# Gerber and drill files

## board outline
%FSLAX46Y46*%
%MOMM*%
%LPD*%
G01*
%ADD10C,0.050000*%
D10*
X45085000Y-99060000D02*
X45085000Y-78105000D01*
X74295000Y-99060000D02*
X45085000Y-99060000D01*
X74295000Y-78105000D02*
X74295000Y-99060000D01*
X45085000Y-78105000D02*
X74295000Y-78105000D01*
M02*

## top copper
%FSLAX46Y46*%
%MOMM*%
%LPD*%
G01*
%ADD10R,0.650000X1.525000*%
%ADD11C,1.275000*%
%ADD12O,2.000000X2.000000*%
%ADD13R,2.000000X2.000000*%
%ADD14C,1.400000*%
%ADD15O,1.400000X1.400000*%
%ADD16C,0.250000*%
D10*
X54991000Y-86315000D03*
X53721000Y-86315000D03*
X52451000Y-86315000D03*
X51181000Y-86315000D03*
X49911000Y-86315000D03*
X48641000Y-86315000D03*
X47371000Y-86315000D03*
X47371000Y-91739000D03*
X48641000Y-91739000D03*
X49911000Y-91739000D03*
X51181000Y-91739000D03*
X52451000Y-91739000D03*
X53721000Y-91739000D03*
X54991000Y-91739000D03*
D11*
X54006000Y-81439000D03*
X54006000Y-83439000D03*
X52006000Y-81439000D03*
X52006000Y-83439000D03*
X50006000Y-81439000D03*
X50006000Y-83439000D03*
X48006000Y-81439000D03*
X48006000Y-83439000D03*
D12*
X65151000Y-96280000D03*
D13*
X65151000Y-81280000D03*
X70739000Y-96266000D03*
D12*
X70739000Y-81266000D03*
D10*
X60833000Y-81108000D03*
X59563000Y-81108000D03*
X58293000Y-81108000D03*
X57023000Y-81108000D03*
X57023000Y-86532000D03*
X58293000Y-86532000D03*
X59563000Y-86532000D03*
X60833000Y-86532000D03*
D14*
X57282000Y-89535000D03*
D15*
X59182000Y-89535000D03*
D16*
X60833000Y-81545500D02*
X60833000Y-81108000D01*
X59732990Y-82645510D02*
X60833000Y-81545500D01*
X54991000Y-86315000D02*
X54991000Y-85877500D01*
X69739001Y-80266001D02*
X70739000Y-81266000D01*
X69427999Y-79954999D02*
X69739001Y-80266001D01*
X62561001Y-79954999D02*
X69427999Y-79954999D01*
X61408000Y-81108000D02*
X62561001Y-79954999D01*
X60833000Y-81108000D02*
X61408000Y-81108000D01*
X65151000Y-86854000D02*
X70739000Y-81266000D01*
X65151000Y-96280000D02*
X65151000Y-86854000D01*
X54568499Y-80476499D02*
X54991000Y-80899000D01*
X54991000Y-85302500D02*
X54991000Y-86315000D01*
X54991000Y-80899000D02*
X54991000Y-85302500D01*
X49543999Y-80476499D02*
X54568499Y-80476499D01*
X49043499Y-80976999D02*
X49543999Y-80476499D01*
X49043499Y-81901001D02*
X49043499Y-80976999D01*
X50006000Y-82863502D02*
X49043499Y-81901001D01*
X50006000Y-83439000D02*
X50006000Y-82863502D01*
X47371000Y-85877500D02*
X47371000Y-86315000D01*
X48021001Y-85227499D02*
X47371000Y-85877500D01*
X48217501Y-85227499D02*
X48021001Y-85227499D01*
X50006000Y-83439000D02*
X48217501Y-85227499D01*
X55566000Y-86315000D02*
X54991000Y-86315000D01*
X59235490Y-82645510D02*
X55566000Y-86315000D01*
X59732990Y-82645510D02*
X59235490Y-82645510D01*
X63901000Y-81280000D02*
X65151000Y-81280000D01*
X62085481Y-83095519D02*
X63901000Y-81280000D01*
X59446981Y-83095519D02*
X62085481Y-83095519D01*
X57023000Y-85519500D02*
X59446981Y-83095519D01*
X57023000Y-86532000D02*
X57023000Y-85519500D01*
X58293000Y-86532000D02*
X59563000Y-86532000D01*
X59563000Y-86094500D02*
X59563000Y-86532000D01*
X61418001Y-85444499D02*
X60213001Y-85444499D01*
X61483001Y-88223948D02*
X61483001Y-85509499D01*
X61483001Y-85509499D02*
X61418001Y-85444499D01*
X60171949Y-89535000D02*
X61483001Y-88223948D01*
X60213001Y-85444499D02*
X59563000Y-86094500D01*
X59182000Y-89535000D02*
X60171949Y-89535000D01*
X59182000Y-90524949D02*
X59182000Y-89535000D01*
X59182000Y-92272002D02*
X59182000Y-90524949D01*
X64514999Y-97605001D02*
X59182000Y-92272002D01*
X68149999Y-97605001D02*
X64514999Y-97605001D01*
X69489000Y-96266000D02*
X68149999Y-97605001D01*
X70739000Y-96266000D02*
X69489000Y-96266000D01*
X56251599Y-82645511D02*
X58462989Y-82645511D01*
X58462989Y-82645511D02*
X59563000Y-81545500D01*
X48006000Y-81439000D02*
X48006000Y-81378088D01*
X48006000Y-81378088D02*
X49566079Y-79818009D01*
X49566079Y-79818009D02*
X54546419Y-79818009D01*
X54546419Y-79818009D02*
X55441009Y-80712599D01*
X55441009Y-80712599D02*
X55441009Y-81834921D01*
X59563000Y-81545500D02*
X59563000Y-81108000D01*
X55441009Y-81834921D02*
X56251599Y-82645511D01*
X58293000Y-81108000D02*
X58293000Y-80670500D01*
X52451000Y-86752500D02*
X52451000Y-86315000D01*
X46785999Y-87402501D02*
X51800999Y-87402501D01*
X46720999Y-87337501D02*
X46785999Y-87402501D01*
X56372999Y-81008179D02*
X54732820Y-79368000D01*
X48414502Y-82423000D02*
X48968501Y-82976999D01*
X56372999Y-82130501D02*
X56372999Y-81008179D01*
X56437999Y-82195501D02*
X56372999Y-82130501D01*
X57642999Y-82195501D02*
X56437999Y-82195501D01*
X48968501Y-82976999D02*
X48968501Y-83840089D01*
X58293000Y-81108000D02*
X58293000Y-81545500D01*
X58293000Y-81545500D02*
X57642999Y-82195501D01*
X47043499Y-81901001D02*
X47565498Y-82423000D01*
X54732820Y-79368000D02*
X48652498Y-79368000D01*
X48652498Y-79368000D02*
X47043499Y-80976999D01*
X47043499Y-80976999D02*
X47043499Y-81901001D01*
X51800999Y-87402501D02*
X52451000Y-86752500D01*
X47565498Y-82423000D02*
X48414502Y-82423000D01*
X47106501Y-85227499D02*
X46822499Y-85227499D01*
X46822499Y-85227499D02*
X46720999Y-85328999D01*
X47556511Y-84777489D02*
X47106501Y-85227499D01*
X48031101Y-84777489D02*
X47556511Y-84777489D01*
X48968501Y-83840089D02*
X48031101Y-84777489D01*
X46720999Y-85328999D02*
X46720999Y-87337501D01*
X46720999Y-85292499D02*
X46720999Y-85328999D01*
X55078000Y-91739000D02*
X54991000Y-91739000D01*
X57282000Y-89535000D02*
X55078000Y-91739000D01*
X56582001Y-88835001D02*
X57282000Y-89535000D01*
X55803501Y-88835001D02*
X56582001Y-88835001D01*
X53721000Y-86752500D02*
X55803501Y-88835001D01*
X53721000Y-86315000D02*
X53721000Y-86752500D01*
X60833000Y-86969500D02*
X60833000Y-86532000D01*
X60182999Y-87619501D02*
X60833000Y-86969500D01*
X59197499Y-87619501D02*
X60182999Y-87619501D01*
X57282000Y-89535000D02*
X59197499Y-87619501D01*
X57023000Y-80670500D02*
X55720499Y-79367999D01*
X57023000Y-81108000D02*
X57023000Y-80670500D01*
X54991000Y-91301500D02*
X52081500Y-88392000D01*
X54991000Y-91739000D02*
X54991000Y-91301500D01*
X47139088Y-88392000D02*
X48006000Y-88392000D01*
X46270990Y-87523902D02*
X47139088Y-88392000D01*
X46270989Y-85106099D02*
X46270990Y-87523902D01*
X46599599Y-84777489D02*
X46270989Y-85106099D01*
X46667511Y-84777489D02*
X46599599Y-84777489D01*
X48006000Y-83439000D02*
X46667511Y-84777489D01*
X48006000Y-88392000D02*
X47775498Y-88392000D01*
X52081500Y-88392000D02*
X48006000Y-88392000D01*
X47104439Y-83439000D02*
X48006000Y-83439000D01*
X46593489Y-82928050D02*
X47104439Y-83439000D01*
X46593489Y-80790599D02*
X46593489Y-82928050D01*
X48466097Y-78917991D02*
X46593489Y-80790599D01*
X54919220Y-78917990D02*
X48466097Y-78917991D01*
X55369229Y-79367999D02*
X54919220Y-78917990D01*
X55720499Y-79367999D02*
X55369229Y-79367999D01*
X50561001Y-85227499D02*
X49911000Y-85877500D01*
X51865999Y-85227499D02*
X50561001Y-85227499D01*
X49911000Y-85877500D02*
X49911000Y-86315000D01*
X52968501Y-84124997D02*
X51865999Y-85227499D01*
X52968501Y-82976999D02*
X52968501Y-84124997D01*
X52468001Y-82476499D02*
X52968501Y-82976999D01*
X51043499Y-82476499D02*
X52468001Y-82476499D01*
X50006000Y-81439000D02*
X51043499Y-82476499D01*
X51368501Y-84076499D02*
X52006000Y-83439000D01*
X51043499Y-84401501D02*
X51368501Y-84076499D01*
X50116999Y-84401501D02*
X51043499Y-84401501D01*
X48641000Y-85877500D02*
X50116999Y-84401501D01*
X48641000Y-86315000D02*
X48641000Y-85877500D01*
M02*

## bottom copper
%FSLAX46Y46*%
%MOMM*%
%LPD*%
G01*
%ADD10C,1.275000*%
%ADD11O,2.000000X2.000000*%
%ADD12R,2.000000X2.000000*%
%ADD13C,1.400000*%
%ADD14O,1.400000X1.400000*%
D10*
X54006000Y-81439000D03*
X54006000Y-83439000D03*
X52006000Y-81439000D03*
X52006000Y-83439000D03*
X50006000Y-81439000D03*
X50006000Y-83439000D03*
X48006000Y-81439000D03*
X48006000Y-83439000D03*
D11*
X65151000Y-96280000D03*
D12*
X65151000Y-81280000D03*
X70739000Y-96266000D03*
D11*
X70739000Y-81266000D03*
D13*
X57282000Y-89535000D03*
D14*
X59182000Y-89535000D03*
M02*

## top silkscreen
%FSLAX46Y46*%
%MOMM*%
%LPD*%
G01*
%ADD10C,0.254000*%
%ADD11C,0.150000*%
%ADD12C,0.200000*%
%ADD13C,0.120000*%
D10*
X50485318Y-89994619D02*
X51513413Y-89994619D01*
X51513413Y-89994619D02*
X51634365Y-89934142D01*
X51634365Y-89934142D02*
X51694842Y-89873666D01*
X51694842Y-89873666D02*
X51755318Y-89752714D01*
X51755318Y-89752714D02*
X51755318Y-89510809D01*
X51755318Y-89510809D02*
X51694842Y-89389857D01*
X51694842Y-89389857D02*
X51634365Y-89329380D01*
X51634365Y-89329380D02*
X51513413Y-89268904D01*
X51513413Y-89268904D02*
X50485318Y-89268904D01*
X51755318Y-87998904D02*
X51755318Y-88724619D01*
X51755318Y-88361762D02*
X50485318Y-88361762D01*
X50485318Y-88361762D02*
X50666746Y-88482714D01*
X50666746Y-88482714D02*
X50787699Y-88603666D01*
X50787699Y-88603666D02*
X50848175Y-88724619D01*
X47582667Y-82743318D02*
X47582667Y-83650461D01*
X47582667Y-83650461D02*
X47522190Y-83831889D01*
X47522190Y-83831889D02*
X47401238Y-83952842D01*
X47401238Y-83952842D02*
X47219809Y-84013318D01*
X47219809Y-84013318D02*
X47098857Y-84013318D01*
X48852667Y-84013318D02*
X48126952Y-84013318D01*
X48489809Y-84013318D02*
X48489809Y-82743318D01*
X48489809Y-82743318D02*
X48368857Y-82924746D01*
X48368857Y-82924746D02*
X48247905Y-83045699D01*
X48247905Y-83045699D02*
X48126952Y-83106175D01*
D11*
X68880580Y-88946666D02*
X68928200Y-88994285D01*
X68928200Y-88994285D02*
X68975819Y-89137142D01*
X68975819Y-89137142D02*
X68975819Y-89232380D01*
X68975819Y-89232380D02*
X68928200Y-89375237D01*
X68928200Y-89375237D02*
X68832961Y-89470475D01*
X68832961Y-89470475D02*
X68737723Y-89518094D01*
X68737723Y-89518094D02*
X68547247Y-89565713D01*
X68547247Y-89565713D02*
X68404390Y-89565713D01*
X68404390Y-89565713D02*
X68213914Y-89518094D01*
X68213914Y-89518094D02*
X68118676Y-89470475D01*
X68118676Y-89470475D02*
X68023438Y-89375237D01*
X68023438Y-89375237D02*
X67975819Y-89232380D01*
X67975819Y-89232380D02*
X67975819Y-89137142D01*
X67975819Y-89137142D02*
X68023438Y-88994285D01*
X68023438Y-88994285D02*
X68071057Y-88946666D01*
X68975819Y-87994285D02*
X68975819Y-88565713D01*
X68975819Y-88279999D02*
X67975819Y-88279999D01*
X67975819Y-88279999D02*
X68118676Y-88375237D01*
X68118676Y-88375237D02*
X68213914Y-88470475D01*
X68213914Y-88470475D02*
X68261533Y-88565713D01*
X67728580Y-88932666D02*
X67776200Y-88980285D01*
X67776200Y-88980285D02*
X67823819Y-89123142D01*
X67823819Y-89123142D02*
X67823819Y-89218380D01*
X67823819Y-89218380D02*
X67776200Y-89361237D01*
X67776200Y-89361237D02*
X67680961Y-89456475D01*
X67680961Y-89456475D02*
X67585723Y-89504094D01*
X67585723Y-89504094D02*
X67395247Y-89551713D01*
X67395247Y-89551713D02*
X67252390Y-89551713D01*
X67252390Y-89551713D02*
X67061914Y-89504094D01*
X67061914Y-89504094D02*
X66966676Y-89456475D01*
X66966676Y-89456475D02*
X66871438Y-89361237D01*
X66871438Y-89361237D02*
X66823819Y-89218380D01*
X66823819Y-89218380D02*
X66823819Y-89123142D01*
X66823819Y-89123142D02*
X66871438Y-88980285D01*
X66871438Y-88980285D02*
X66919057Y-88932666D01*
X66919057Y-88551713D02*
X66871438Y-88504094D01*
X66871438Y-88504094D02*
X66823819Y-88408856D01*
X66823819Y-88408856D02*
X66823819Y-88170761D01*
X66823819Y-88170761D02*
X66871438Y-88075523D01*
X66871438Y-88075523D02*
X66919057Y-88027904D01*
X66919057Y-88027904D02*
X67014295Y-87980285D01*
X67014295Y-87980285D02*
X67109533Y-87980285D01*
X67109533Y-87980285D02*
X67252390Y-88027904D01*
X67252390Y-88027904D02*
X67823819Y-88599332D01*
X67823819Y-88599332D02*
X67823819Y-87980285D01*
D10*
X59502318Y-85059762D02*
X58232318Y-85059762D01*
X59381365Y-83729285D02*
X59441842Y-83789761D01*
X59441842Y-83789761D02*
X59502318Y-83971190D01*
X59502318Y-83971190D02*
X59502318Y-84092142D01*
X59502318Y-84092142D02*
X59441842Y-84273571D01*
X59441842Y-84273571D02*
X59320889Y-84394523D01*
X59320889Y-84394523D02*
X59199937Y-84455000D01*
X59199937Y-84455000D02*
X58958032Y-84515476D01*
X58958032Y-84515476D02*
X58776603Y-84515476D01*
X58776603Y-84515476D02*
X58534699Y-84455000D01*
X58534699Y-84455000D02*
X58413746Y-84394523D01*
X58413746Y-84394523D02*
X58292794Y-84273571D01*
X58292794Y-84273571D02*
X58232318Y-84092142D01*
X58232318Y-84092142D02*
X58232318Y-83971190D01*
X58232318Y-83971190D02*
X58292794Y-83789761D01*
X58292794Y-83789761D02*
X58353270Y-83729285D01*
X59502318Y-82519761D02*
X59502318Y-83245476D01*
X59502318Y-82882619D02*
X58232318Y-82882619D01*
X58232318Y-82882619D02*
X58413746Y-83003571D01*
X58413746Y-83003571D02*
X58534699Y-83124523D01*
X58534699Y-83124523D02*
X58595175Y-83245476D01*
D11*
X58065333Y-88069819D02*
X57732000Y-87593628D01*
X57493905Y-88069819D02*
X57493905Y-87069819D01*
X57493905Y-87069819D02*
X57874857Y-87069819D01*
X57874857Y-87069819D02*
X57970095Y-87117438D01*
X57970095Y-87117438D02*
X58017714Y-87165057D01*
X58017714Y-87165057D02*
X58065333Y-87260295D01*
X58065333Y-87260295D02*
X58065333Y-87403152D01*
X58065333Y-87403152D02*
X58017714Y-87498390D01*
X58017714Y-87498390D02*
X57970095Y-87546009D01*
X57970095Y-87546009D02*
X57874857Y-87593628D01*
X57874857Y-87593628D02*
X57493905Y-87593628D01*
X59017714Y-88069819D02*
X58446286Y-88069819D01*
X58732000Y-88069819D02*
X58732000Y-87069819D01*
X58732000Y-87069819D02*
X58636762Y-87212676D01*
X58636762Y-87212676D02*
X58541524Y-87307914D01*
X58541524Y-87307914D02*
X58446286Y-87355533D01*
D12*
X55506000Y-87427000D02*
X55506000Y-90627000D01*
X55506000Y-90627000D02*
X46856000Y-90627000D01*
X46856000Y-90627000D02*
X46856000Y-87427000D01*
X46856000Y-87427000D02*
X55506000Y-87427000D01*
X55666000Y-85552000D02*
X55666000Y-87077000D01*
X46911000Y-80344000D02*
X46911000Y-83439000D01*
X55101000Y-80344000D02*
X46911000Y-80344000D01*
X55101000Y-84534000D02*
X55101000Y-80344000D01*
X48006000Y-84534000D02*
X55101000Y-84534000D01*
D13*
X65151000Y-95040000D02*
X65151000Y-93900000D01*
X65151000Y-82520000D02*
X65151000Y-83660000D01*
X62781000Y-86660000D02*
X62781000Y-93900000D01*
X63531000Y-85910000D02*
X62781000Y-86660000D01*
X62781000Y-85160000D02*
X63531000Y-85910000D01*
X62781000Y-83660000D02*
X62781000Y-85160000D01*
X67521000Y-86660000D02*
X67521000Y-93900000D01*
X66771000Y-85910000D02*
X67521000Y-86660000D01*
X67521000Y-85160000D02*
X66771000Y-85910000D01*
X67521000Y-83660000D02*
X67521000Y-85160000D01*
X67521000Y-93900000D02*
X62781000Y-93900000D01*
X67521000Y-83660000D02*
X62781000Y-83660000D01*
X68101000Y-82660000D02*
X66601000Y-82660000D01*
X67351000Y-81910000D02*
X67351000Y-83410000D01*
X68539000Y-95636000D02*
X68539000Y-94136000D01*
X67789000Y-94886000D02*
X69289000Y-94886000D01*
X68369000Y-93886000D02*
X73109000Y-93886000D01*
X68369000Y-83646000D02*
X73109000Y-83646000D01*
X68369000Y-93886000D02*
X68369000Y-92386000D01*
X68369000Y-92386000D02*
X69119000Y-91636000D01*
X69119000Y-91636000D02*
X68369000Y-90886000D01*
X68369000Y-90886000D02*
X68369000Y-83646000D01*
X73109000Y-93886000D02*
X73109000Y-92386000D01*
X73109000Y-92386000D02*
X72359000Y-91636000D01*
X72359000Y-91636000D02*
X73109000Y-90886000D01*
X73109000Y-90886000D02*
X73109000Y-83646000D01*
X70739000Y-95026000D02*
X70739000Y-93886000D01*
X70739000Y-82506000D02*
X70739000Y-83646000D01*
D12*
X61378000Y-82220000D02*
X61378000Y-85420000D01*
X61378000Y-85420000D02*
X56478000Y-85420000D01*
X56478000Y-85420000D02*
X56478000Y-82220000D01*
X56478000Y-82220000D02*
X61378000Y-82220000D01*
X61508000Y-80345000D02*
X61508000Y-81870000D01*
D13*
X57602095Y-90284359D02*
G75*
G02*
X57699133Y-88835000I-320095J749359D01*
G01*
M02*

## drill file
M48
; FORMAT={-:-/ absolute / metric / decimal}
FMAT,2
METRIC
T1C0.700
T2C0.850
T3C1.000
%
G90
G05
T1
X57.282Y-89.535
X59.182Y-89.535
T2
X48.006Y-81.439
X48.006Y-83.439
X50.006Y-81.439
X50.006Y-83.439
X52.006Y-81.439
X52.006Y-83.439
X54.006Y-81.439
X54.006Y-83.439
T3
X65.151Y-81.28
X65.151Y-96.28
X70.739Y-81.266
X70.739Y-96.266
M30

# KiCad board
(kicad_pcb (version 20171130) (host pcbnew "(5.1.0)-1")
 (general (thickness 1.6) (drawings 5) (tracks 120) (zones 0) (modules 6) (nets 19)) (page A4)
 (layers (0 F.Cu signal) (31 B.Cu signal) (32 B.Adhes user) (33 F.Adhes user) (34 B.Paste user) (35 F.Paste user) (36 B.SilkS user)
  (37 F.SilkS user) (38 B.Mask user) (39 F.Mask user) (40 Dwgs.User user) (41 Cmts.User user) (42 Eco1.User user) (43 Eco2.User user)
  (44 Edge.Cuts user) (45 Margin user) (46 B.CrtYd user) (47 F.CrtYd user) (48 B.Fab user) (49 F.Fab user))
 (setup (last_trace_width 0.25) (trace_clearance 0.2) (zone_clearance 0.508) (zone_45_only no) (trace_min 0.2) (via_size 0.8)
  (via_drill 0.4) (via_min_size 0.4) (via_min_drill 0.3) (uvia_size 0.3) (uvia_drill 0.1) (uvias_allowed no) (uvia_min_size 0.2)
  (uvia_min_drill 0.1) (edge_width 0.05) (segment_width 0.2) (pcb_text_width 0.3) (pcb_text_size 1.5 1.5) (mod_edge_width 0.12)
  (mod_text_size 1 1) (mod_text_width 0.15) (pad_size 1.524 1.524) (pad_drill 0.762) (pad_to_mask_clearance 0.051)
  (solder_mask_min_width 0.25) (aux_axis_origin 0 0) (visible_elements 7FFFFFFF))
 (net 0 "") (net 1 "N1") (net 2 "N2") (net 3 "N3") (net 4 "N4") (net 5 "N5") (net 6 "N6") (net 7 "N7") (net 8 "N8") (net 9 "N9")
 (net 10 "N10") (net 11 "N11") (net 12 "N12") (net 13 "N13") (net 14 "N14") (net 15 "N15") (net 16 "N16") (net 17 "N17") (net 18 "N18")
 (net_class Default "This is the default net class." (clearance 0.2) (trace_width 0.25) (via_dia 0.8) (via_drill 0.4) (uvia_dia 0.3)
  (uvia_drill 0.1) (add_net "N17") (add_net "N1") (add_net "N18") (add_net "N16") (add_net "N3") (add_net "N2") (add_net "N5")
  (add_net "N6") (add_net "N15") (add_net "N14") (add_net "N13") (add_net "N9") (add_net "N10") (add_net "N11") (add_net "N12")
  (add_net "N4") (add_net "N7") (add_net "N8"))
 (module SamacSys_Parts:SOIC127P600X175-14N (layer F.Cu) (at 51.181 89.027 270)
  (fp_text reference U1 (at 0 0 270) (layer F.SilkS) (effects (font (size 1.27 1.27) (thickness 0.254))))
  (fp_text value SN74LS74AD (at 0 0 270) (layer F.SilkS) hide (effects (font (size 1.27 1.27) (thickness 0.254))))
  (fp_line (start -1.6 -4.325) (end 1.6 -4.325) (layer F.SilkS) (width 0.2))
  (fp_line (start 1.6 -4.325) (end 1.6 4.325) (layer F.SilkS) (width 0.2))
  (fp_line (start 1.6 4.325) (end -1.6 4.325) (layer F.SilkS) (width 0.2))
  (fp_line (start -1.6 4.325) (end -1.6 -4.325) (layer F.SilkS) (width 0.2))
  (fp_line (start -3.475 -4.485) (end -1.95 -4.485) (layer F.SilkS) (width 0.2))
  (pad 1 smd rect (at -2.712 -3.81) (size 0.65 1.525) (layers F.Cu F.Paste F.Mask) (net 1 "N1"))
  (pad 2 smd rect (at -2.712 -2.54) (size 0.65 1.525) (layers F.Cu F.Paste F.Mask) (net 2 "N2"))
  (pad 3 smd rect (at -2.712 -1.27) (size 0.65 1.525) (layers F.Cu F.Paste F.Mask) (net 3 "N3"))
  (pad 4 smd rect (at -2.712 0) (size 0.65 1.525) (layers F.Cu F.Paste F.Mask) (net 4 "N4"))
  (pad 5 smd rect (at -2.712 1.27) (size 0.65 1.525) (layers F.Cu F.Paste F.Mask) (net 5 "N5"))
  (pad 6 smd rect (at -2.712 2.54) (size 0.65 1.525) (layers F.Cu F.Paste F.Mask) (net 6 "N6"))
  (pad 7 smd rect (at -2.712 3.81) (size 0.65 1.525) (layers F.Cu F.Paste F.Mask) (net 1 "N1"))
  (pad 8 smd rect (at 2.712 3.81) (size 0.65 1.525) (layers F.Cu F.Paste F.Mask) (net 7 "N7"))
  (pad 9 smd rect (at 2.712 2.54) (size 0.65 1.525) (layers F.Cu F.Paste F.Mask) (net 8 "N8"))
  (pad 10 smd rect (at 2.712 1.27) (size 0.65 1.525) (layers F.Cu F.Paste F.Mask) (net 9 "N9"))
  (pad 11 smd rect (at 2.712 0) (size 0.65 1.525) (layers F.Cu F.Paste F.Mask) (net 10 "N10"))
  (pad 12 smd rect (at 2.712 -1.27) (size 0.65 1.525) (layers F.Cu F.Paste F.Mask) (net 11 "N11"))
  (pad 13 smd rect (at 2.712 -2.54) (size 0.65 1.525) (layers F.Cu F.Paste F.Mask) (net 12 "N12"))
  (pad 14 smd rect (at 2.712 -3.81) (size 0.65 1.525) (layers F.Cu F.Paste F.Mask) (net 2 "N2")))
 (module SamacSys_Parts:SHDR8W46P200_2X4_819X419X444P (layer F.Cu) (at 48.006 83.439)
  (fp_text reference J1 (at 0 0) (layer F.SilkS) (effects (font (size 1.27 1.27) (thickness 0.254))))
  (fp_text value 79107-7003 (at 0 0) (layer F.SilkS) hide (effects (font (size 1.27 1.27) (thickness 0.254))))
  (fp_line (start -1.095 -3.095) (end -1.095 0) (layer F.SilkS) (width 0.2))
  (fp_line (start 7.095 -3.095) (end -1.095 -3.095) (layer F.SilkS) (width 0.2))
  (fp_line (start 7.095 1.095) (end 7.095 -3.095) (layer F.SilkS) (width 0.2))
  (fp_line (start 0 1.095) (end 7.095 1.095) (layer F.SilkS) (width 0.2))
  (pad 8 thru_hole circle (at 6 -2) (size 1.275 1.275) (drill 0.85) (layers *.Cu *.Mask) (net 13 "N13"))
  (pad 7 thru_hole circle (at 6 0) (size 1.275 1.275) (drill 0.85) (layers *.Cu *.Mask) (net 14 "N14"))
  (pad 6 thru_hole circle (at 4 -2) (size 1.275 1.275) (drill 0.85) (layers *.Cu *.Mask) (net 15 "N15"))
  (pad 5 thru_hole circle (at 4 0) (size 1.275 1.275) (drill 0.85) (layers *.Cu *.Mask) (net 6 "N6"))
  (pad 4 thru_hole circle (at 2 -2) (size 1.275 1.275) (drill 0.85) (layers *.Cu *.Mask) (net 5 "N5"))
  (pad 3 thru_hole circle (at 2 0) (size 1.275 1.275) (drill 0.85) (layers *.Cu *.Mask) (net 1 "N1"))
  (pad 2 thru_hole circle (at 0 -2) (size 1.275 1.275) (drill 0.85) (layers *.Cu *.Mask) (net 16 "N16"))
  (pad 1 thru_hole circle (at 0 0) (size 1.275 1.275) (drill 0.85) (layers *.Cu *.Mask) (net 2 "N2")))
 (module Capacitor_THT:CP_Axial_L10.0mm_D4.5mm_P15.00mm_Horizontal (layer F.Cu) (at 65.151 81.28 270)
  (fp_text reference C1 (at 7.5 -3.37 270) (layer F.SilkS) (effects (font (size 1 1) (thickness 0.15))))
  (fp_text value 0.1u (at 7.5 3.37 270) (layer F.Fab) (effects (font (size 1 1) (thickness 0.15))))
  (fp_line (start 13.76 0) (end 12.62 0) (layer F.SilkS) (width 0.12))
  (fp_line (start 1.24 0) (end 2.38 0) (layer F.SilkS) (width 0.12))
  (fp_line (start 5.38 2.37) (end 12.62 2.37) (layer F.SilkS) (width 0.12))
  (fp_line (start 4.63 1.62) (end 5.38 2.37) (layer F.SilkS) (width 0.12))
  (fp_line (start 3.88 2.37) (end 4.63 1.62) (layer F.SilkS) (width 0.12))
  (fp_line (start 2.38 2.37) (end 3.88 2.37) (layer F.SilkS) (width 0.12))
  (fp_line (start 5.38 -2.37) (end 12.62 -2.37) (layer F.SilkS) (width 0.12))
  (fp_line (start 4.63 -1.62) (end 5.38 -2.37) (layer F.SilkS) (width 0.12))
  (fp_line (start 3.88 -2.37) (end 4.63 -1.62) (layer F.SilkS) (width 0.12))
  (fp_line (start 2.38 -2.37) (end 3.88 -2.37) (layer F.SilkS) (width 0.12))
  (fp_line (start 12.62 -2.37) (end 12.62 2.37) (layer F.SilkS) (width 0.12))
  (fp_line (start 2.38 -2.37) (end 2.38 2.37) (layer F.SilkS) (width 0.12))
  (fp_line (start 1.38 -2.95) (end 1.38 -1.45) (layer F.SilkS) (width 0.12))
  (fp_line (start 0.63 -2.2) (end 2.13 -2.2) (layer F.SilkS) (width 0.12))
  (pad 2 thru_hole oval (at 15 0 270) (size 2 2) (drill 1) (layers *.Cu *.Mask) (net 1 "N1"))
  (pad 1 thru_hole rect (at 0 0 270) (size 2 2) (drill 1) (layers *.Cu *.Mask) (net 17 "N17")))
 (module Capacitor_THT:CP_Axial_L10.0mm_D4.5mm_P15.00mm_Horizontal (layer F.Cu) (at 70.739 96.266 90)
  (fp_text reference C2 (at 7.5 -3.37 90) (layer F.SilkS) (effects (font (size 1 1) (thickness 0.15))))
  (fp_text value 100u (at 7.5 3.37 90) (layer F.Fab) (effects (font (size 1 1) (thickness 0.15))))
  (fp_line (start 0.63 -2.2) (end 2.13 -2.2) (layer F.SilkS) (width 0.12))
  (fp_line (start 1.38 -2.95) (end 1.38 -1.45) (layer F.SilkS) (width 0.12))
  (fp_line (start 2.38 -2.37) (end 2.38 2.37) (layer F.SilkS) (width 0.12))
  (fp_line (start 12.62 -2.37) (end 12.62 2.37) (layer F.SilkS) (width 0.12))
  (fp_line (start 2.38 -2.37) (end 3.88 -2.37) (layer F.SilkS) (width 0.12))
  (fp_line (start 3.88 -2.37) (end 4.63 -1.62) (layer F.SilkS) (width 0.12))
  (fp_line (start 4.63 -1.62) (end 5.38 -2.37) (layer F.SilkS) (width 0.12))
  (fp_line (start 5.38 -2.37) (end 12.62 -2.37) (layer F.SilkS) (width 0.12))
  (fp_line (start 2.38 2.37) (end 3.88 2.37) (layer F.SilkS) (width 0.12))
  (fp_line (start 3.88 2.37) (end 4.63 1.62) (layer F.SilkS) (width 0.12))
  (fp_line (start 4.63 1.62) (end 5.38 2.37) (layer F.SilkS) (width 0.12))
  (fp_line (start 5.38 2.37) (end 12.62 2.37) (layer F.SilkS) (width 0.12))
  (fp_line (start 1.24 0) (end 2.38 0) (layer F.SilkS) (width 0.12))
  (fp_line (start 13.76 0) (end 12.62 0) (layer F.SilkS) (width 0.12))
  (pad 1 thru_hole rect (at 0 0 90) (size 2 2) (drill 1) (layers *.Cu *.Mask) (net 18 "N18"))
  (pad 2 thru_hole oval (at 15 0 90) (size 2 2) (drill 1) (layers *.Cu *.Mask) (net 1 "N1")))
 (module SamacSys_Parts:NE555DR (layer F.Cu) (at 58.928 83.82 270)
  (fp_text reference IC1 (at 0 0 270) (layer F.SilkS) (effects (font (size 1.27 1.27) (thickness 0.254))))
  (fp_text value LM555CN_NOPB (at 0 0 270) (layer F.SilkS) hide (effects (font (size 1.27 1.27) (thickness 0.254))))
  (fp_line (start -1.6 -2.45) (end 1.6 -2.45) (layer F.SilkS) (width 0.2))
  (fp_line (start 1.6 -2.45) (end 1.6 2.45) (layer F.SilkS) (width 0.2))
  (fp_line (start 1.6 2.45) (end -1.6 2.45) (layer F.SilkS) (width 0.2))
  (fp_line (start -1.6 2.45) (end -1.6 -2.45) (layer F.SilkS) (width 0.2))
  (fp_line (start -3.475 -2.58) (end -1.95 -2.58) (layer F.SilkS) (width 0.2))
  (pad 1 smd rect (at -2.712 -1.905) (size 0.65 1.525) (layers F.Cu F.Paste) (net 1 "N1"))
  (pad 2 smd rect (at -2.712 -0.635) (size 0.65 1.525) (layers F.Cu F.Paste) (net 16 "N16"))
  (pad 3 smd rect (at -2.712 0.635) (size 0.65 1.525) (layers F.Cu F.Paste) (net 3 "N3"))
  (pad 4 smd rect (at -2.712 1.905) (size 0.65 1.525) (layers F.Cu F.Paste) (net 2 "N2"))
  (pad 5 smd rect (at 2.712 1.905) (size 0.65 1.525) (layers F.Cu F.Paste) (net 17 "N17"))
  (pad 6 smd rect (at 2.712 0.635) (size 0.65 1.525) (layers F.Cu F.Paste) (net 18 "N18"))
  (pad 7 smd rect (at 2.712 -0.635) (size 0.65 1.525) (layers F.Cu F.Paste) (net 18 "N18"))
  (pad 8 smd rect (at 2.712 -1.905) (size 0.65 1.525) (layers F.Cu F.Paste) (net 2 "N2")))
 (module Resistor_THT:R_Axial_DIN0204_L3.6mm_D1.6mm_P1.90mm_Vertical (layer F.Cu) (at 57.282 89.535)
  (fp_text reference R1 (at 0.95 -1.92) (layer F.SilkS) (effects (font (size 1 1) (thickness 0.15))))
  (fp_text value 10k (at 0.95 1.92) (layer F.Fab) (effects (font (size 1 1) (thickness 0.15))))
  (fp_arc (start 0 0) (end 0.417133 -0.7) (angle -233.92106) (layer F.SilkS) (width 0.12))
  (pad 1 thru_hole circle (at 0 0) (size 1.4 1.4) (drill 0.7) (layers *.Cu *.Mask) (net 2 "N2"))
  (pad 2 thru_hole oval (at 1.9 0) (size 1.4 1.4) (drill 0.7) (layers *.Cu *.Mask) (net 18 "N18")))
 (gr_line (start 45.085 99.06) (end 45.085 78.105) (layer Edge.Cuts) (width 0.05))
 (gr_line (start 74.295 99.06) (end 45.085 99.06) (layer Edge.Cuts) (width 0.05))
 (gr_line (start 74.295 78.105) (end 74.295 99.06) (layer Edge.Cuts) (width 0.05))
 (gr_line (start 45.085 78.105) (end 74.295 78.105) (layer Edge.Cuts) (width 0.05))
 (segment (start 60.833 81.5455) (end 60.833 81.108) (width 0.25) (layer F.Cu) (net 1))
 (segment (start 59.73299 82.64551) (end 60.833 81.5455) (width 0.25) (layer F.Cu) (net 1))
 (segment (start 54.991 86.315) (end 54.991 85.8775) (width 0.25) (layer F.Cu) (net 1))
 (segment (start 69.739001 80.266001) (end 70.739 81.266) (width 0.25) (layer F.Cu) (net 1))
 (segment (start 69.427999 79.954999) (end 69.739001 80.266001) (width 0.25) (layer F.Cu) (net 1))
 (segment (start 62.561001 79.954999) (end 69.427999 79.954999) (width 0.25) (layer F.Cu) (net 1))
 (segment (start 61.408 81.108) (end 62.561001 79.954999) (width 0.25) (layer F.Cu) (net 1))
 (segment (start 60.833 81.108) (end 61.408 81.108) (width 0.25) (layer F.Cu) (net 1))
 (segment (start 65.151 86.854) (end 70.739 81.266) (width 0.25) (layer F.Cu) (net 1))
 (segment (start 65.151 96.28) (end 65.151 86.854) (width 0.25) (layer F.Cu) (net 1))
 (segment (start 54.568499 80.476499) (end 54.991 80.899) (width 0.25) (layer F.Cu) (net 1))
 (segment (start 54.991 85.3025) (end 54.991 86.315) (width 0.25) (layer F.Cu) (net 1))
 (segment (start 54.991 80.899) (end 54.991 85.3025) (width 0.25) (layer F.Cu) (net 1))
 (segment (start 49.543999 80.476499) (end 54.568499 80.476499) (width 0.25) (layer F.Cu) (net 1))
 (segment (start 49.043499 80.976999) (end 49.543999 80.476499) (width 0.25) (layer F.Cu) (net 1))
 (segment (start 49.043499 81.901001) (end 49.043499 80.976999) (width 0.25) (layer F.Cu) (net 1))
 (segment (start 50.006 82.863502) (end 49.043499 81.901001) (width 0.25) (layer F.Cu) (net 1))
 (segment (start 50.006 83.439) (end 50.006 82.863502) (width 0.25) (layer F.Cu) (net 1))
 (segment (start 47.371 85.8775) (end 47.371 86.315) (width 0.25) (layer F.Cu) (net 1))
 (segment (start 48.021001 85.227499) (end 47.371 85.8775) (width 0.25) (layer F.Cu) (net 1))
 (segment (start 48.217501 85.227499) (end 48.021001 85.227499) (width 0.25) (layer F.Cu) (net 1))
 (segment (start 50.006 83.439) (end 48.217501 85.227499) (width 0.25) (layer F.Cu) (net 1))
 (segment (start 55.566 86.315) (end 54.991 86.315) (width 0.25) (layer F.Cu) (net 1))
 (segment (start 59.23549 82.64551) (end 55.566 86.315) (width 0.25) (layer F.Cu) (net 1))
 (segment (start 59.73299 82.64551) (end 59.23549 82.64551) (width 0.25) (layer F.Cu) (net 1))
 (segment (start 63.901 81.28) (end 65.151 81.28) (width 0.25) (layer F.Cu) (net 17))
 (segment (start 62.085481 83.095519) (end 63.901 81.28) (width 0.25) (layer F.Cu) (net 17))
 (segment (start 59.446981 83.095519) (end 62.085481 83.095519) (width 0.25) (layer F.Cu) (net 17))
 (segment (start 57.023 85.5195) (end 59.446981 83.095519) (width 0.25) (layer F.Cu) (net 17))
 (segment (start 57.023 86.532) (end 57.023 85.5195) (width 0.25) (layer F.Cu) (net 17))
 (segment (start 58.293 86.532) (end 59.563 86.532) (width 0.25) (layer F.Cu) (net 18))
 (segment (start 59.563 86.0945) (end 59.563 86.532) (width 0.25) (layer F.Cu) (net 18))
 (segment (start 61.418001 85.444499) (end 60.213001 85.444499) (width 0.25) (layer F.Cu) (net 18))
 (segment (start 61.483001 88.223948) (end 61.483001 85.509499) (width 0.25) (layer F.Cu) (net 18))
 (segment (start 61.483001 85.509499) (end 61.418001 85.444499) (width 0.25) (layer F.Cu) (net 18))
 (segment (start 60.171949 89.535) (end 61.483001 88.223948) (width 0.25) (layer F.Cu) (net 18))
 (segment (start 60.213001 85.444499) (end 59.563 86.0945) (width 0.25) (layer F.Cu) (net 18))
 (segment (start 59.182 89.535) (end 60.171949 89.535) (width 0.25) (layer F.Cu) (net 18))
 (segment (start 59.182 90.524949) (end 59.182 89.535) (width 0.25) (layer F.Cu) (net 18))
 (segment (start 59.182 92.272002) (end 59.182 90.524949) (width 0.25) (layer F.Cu) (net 18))
 (segment (start 64.514999 97.605001) (end 59.182 92.272002) (width 0.25) (layer F.Cu) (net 18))
 (segment (start 68.149999 97.605001) (end 64.514999 97.605001) (width 0.25) (layer F.Cu) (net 18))
 (segment (start 69.489 96.266) (end 68.149999 97.605001) (width 0.25) (layer F.Cu) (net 18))
 (segment (start 70.739 96.266) (end 69.489 96.266) (width 0.25) (layer F.Cu) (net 18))
 (segment (start 56.251599 82.645511) (end 58.462989 82.645511) (width 0.25) (layer F.Cu) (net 16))
 (segment (start 58.462989 82.645511) (end 59.563 81.5455) (width 0.25) (layer F.Cu) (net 16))
 (segment (start 48.006 81.439) (end 48.006 81.378088) (width 0.25) (layer F.Cu) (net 16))
 (segment (start 48.006 81.378088) (end 49.566079 79.818009) (width 0.25) (layer F.Cu) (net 16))
 (segment (start 49.566079 79.818009) (end 54.546419 79.818009) (width 0.25) (layer F.Cu) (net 16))
 (segment (start 54.546419 79.818009) (end 55.441009 80.712599) (width 0.25) (layer F.Cu) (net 16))
 (segment (start 55.441009 80.712599) (end 55.441009 81.834921) (width 0.25) (layer F.Cu) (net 16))
 (segment (start 59.563 81.5455) (end 59.563 81.108) (width 0.25) (layer F.Cu) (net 16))
 (segment (start 55.441009 81.834921) (end 56.251599 82.645511) (width 0.25) (layer F.Cu) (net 16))
 (segment (start 58.293 81.108) (end 58.293 80.6705) (width 0.25) (layer F.Cu) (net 3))
 (segment (start 52.451 86.7525) (end 52.451 86.315) (width 0.25) (layer F.Cu) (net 3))
 (segment (start 46.785999 87.402501) (end 51.800999 87.402501) (width 0.25) (layer F.Cu) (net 3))
 (segment (start 46.720999 87.337501) (end 46.785999 87.402501) (width 0.25) (layer F.Cu) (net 3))
 (segment (start 56.372999 81.008179) (end 54.73282 79.368) (width 0.25) (layer F.Cu) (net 3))
 (segment (start 48.414502 82.423) (end 48.968501 82.976999) (width 0.25) (layer F.Cu) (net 3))
 (segment (start 56.372999 82.130501) (end 56.372999 81.008179) (width 0.25) (layer F.Cu) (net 3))
 (segment (start 56.437999 82.195501) (end 56.372999 82.130501) (width 0.25) (layer F.Cu) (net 3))
 (segment (start 57.642999 82.195501) (end 56.437999 82.195501) (width 0.25) (layer F.Cu) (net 3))
 (segment (start 48.968501 82.976999) (end 48.968501 83.840089) (width 0.25) (layer F.Cu) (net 3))
 (segment (start 58.293 81.108) (end 58.293 81.5455) (width 0.25) (layer F.Cu) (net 3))
 (segment (start 58.293 81.5455) (end 57.642999 82.195501) (width 0.25) (layer F.Cu) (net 3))
 (segment (start 47.043499 81.901001) (end 47.565498 82.423) (width 0.25) (layer F.Cu) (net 3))
 (segment (start 54.73282 79.368) (end 48.652498 79.368) (width 0.25) (layer F.Cu) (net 3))
 (segment (start 48.652498 79.368) (end 47.043499 80.976999) (width 0.25) (layer F.Cu) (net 3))
 (segment (start 47.043499 80.976999) (end 47.043499 81.901001) (width 0.25) (layer F.Cu) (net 3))
 (segment (start 51.800999 87.402501) (end 52.451 86.7525) (width 0.25) (layer F.Cu) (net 3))
 (segment (start 47.565498 82.423) (end 48.414502 82.423) (width 0.25) (layer F.Cu) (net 3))
 (segment (start 47.106501 85.227499) (end 46.822499 85.227499) (width 0.25) (layer F.Cu) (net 3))
 (segment (start 46.822499 85.227499) (end 46.720999 85.328999) (width 0.25) (layer F.Cu) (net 3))
 (segment (start 47.556511 84.777489) (end 47.106501 85.227499) (width 0.25) (layer F.Cu) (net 3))
 (segment (start 48.031101 84.777489) (end 47.556511 84.777489) (width 0.25) (layer F.Cu) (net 3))
 (segment (start 48.968501 83.840089) (end 48.031101 84.777489) (width 0.25) (layer F.Cu) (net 3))
 (segment (start 46.720999 85.328999) (end 46.720999 87.337501) (width 0.25) (layer F.Cu) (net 3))
 (segment (start 46.720999 85.292499) (end 46.720999 85.328999) (width 0.25) (layer F.Cu) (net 3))
 (segment (start 55.078 91.739) (end 54.991 91.739) (width 0.25) (layer F.Cu) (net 2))
 (segment (start 57.282 89.535) (end 55.078 91.739) (width 0.25) (layer F.Cu) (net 2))
 (segment (start 56.582001 88.835001) (end 57.282 89.535) (width 0.25) (layer F.Cu) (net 2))
 (segment (start 55.803501 88.835001) (end 56.582001 88.835001) (width 0.25) (layer F.Cu) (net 2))
 (segment (start 53.721 86.7525) (end 55.803501 88.835001) (width 0.25) (layer F.Cu) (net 2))
 (segment (start 53.721 86.315) (end 53.721 86.7525) (width 0.25) (layer F.Cu) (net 2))
 (segment (start 60.833 86.9695) (end 60.833 86.532) (width 0.25) (layer F.Cu) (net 2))
 (segment (start 60.182999 87.619501) (end 60.833 86.9695) (width 0.25) (layer F.Cu) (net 2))
 (segment (start 59.197499 87.619501) (end 60.182999 87.619501) (width 0.25) (layer F.Cu) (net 2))
 (segment (start 57.282 89.535) (end 59.197499 87.619501) (width 0.25) (layer F.Cu) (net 2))
 (segment (start 57.023 80.6705) (end 55.720499 79.367999) (width 0.25) (layer F.Cu) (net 2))
 (segment (start 57.023 81.108) (end 57.023 80.6705) (width 0.25) (layer F.Cu) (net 2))
 (segment (start 54.991 91.3015) (end 52.0815 88.392) (width 0.25) (layer F.Cu) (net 2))
 (segment (start 54.991 91.739) (end 54.991 91.3015) (width 0.25) (layer F.Cu) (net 2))
 (segment (start 47.139088 88.392) (end 48.006 88.392) (width 0.25) (layer F.Cu) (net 2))
 (segment (start 46.27099 87.523902) (end 47.139088 88.392) (width 0.25) (layer F.Cu) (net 2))
 (segment (start 46.270989 85.106099) (end 46.27099 87.523902) (width 0.25) (layer F.Cu) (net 2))
 (segment (start 46.599599 84.777489) (end 46.270989 85.106099) (width 0.25) (layer F.Cu) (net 2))
 (segment (start 46.667511 84.777489) (end 46.599599 84.777489) (width 0.25) (layer F.Cu) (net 2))
 (segment (start 48.006 83.439) (end 46.667511 84.777489) (width 0.25) (layer F.Cu) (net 2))
 (segment (start 48.006 88.392) (end 47.775498 88.392) (width 0.25) (layer F.Cu) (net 2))
 (segment (start 52.0815 88.392) (end 48.006 88.392) (width 0.25) (layer F.Cu) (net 2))
 (segment (start 47.104439 83.439) (end 48.006 83.439) (width 0.25) (layer F.Cu) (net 2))
 (segment (start 46.593489 82.92805) (end 47.104439 83.439) (width 0.25) (layer F.Cu) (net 2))
 (segment (start 46.593489 80.790599) (end 46.593489 82.92805) (width 0.25) (layer F.Cu) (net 2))
 (segment (start 48.466097 78.917991) (end 46.593489 80.790599) (width 0.25) (layer F.Cu) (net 2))
 (segment (start 54.91922 78.91799) (end 48.466097 78.917991) (width 0.25) (layer F.Cu) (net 2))
 (segment (start 55.369229 79.367999) (end 54.91922 78.91799) (width 0.25) (layer F.Cu) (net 2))
 (segment (start 55.720499 79.367999) (end 55.369229 79.367999) (width 0.25) (layer F.Cu) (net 2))
 (segment (start 50.561001 85.227499) (end 49.911 85.8775) (width 0.25) (layer F.Cu) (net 5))
 (segment (start 51.865999 85.227499) (end 50.561001 85.227499) (width 0.25) (layer F.Cu) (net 5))
 (segment (start 49.911 85.8775) (end 49.911 86.315) (width 0.25) (layer F.Cu) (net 5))
 (segment (start 52.968501 84.124997) (end 51.865999 85.227499) (width 0.25) (layer F.Cu) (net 5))
 (segment (start 52.968501 82.976999) (end 52.968501 84.124997) (width 0.25) (layer F.Cu) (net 5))
 (segment (start 52.468001 82.476499) (end 52.968501 82.976999) (width 0.25) (layer F.Cu) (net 5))
 (segment (start 51.043499 82.476499) (end 52.468001 82.476499) (width 0.25) (layer F.Cu) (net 5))
 (segment (start 50.006 81.439) (end 51.043499 82.476499) (width 0.25) (layer F.Cu) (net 5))
 (segment (start 51.368501 84.076499) (end 52.006 83.439) (width 0.25) (layer F.Cu) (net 6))
 (segment (start 51.043499 84.401501) (end 51.368501 84.076499) (width 0.25) (layer F.Cu) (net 6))
 (segment (start 50.116999 84.401501) (end 51.043499 84.401501) (width 0.25) (layer F.Cu) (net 6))
 (segment (start 48.641 85.8775) (end 50.116999 84.401501) (width 0.25) (layer F.Cu) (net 6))
 (segment (start 48.641 86.315) (end 48.641 85.8775) (width 0.25) (layer F.Cu) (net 6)))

